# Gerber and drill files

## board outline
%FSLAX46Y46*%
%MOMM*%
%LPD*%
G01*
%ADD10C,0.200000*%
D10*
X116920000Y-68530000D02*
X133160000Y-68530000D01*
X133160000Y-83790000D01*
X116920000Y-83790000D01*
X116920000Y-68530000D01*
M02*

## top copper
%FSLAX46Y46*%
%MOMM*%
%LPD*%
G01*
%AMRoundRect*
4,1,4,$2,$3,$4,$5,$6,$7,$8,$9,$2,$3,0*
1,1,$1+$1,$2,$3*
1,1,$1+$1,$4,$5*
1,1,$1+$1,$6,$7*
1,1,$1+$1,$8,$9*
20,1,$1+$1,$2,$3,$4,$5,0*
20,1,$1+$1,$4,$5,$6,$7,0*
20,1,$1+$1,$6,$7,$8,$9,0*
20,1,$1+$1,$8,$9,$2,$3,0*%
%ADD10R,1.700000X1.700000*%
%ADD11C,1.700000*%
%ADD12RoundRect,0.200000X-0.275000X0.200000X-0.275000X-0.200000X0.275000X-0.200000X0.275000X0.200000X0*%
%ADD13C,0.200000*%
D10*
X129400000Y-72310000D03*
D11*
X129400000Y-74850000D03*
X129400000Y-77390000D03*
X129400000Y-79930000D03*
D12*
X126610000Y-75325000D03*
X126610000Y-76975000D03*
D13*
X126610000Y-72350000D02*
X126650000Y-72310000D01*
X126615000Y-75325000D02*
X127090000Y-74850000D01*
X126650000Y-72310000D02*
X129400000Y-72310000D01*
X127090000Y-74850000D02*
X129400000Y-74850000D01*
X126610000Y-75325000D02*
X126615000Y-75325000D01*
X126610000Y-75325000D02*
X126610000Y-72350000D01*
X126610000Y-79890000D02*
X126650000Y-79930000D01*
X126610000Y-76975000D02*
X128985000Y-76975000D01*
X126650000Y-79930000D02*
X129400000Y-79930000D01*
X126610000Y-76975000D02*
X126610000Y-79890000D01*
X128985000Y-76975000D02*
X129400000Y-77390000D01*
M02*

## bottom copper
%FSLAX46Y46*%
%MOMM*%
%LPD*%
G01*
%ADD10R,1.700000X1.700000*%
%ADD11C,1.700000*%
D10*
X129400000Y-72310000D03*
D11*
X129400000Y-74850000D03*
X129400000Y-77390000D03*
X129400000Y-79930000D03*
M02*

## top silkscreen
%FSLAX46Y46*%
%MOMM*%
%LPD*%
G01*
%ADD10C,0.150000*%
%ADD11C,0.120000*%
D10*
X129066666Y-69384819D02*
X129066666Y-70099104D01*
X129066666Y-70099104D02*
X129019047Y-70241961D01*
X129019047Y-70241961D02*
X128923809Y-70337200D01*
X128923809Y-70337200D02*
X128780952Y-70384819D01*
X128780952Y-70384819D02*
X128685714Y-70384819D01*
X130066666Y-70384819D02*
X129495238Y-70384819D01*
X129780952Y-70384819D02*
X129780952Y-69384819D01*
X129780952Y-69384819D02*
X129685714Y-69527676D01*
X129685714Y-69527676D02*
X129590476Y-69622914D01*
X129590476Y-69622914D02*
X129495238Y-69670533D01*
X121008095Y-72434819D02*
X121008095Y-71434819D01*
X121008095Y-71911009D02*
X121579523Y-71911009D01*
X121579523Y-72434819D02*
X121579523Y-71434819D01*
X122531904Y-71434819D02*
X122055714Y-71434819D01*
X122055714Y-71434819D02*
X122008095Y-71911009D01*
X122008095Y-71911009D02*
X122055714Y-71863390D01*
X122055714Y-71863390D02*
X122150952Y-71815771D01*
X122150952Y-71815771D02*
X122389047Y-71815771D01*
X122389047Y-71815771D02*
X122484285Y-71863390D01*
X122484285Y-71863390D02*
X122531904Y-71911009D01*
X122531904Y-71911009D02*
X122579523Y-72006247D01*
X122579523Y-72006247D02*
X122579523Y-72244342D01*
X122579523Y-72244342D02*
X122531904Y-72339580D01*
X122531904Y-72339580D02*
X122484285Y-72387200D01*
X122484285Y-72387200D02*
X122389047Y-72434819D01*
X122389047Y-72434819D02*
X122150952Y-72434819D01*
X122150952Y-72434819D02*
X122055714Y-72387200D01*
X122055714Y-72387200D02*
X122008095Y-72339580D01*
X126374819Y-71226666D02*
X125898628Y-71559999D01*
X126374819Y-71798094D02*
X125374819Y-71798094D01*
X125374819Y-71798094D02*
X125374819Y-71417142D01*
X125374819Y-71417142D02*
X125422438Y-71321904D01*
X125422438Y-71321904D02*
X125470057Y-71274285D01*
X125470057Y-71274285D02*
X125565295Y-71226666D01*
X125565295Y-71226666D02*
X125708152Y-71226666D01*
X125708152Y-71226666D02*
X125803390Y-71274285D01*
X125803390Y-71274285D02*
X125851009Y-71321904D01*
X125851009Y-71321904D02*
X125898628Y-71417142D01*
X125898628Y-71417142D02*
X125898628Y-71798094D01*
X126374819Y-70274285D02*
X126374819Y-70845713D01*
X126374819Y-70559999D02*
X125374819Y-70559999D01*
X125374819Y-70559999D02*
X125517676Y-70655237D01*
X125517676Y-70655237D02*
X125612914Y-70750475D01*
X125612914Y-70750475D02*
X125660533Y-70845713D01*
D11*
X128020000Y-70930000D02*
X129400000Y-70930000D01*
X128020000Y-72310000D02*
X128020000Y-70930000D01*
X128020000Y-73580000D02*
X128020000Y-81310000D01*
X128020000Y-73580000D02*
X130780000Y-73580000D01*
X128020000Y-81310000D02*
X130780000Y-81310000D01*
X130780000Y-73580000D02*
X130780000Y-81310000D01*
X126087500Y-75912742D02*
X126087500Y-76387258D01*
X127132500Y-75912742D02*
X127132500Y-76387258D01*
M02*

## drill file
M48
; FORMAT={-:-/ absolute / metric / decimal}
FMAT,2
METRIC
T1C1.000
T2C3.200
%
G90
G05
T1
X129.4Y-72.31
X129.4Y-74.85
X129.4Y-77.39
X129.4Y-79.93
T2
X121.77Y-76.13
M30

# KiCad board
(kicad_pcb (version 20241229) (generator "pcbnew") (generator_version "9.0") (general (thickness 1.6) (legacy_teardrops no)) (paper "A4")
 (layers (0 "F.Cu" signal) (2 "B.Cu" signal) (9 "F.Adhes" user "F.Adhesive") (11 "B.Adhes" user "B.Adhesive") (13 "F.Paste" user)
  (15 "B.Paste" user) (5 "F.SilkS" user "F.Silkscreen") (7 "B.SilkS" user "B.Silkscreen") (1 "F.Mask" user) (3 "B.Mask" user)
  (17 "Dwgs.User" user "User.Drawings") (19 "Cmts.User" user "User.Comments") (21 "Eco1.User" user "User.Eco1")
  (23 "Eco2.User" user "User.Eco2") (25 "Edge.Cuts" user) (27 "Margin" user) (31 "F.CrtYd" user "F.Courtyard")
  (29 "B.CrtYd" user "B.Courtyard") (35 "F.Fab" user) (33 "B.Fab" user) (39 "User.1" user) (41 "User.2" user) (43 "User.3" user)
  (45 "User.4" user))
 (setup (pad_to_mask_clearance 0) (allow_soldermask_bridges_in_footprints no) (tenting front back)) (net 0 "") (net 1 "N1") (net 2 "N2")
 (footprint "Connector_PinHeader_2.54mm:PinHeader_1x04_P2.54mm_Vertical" (layer "F.Cu") (at 129.4 72.31)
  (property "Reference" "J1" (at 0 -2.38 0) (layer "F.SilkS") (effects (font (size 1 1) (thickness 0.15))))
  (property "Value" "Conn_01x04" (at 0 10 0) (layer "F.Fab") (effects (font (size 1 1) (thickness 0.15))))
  (fp_line (start -1.38 -1.38) (end 0 -1.38) (stroke (width 0.12) (type solid)) (layer "F.SilkS"))
  (fp_line (start -1.38 0) (end -1.38 -1.38) (stroke (width 0.12) (type solid)) (layer "F.SilkS"))
  (fp_line (start -1.38 1.27) (end -1.38 9) (stroke (width 0.12) (type solid)) (layer "F.SilkS"))
  (fp_line (start -1.38 1.27) (end 1.38 1.27) (stroke (width 0.12) (type solid)) (layer "F.SilkS"))
  (fp_line (start -1.38 9) (end 1.38 9) (stroke (width 0.12) (type solid)) (layer "F.SilkS"))
  (fp_line (start 1.38 1.27) (end 1.38 9) (stroke (width 0.12) (type solid)) (layer "F.SilkS"))
  (pad "1" thru_hole rect (at 0 0) (size 1.7 1.7) (drill 1) (layers "*.Cu" "*.Mask") (remove_unused_layers no) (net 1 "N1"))
  (pad "2" thru_hole circle (at 0 2.54) (size 1.7 1.7) (drill 1) (layers "*.Cu" "*.Mask") (remove_unused_layers no) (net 1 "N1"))
  (pad "3" thru_hole circle (at 0 5.08) (size 1.7 1.7) (drill 1) (layers "*.Cu" "*.Mask") (remove_unused_layers no) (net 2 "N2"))
  (pad "4" thru_hole circle (at 0 7.62) (size 1.7 1.7) (drill 1) (layers "*.Cu" "*.Mask") (remove_unused_layers no) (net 2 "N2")))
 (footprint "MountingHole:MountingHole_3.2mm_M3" (layer "F.Cu") (at 121.77 76.13)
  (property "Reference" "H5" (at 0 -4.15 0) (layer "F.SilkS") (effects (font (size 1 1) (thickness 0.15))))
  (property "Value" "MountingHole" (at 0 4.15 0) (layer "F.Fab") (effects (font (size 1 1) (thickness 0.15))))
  (pad "" np_thru_hole circle (at 0 0) (size 3.2 3.2) (drill 3.2) (layers "*.Cu" "*.Mask")))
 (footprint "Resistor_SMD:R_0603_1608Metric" (layer "F.Cu") (at 126.61 76.15 -90)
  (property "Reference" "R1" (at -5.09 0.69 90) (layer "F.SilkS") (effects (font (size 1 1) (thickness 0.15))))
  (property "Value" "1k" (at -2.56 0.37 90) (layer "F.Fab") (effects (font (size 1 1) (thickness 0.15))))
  (fp_line (start -0.237258 0.5225) (end 0.237258 0.5225) (stroke (width 0.12) (type solid)) (layer "F.SilkS"))
  (fp_line (start -0.237258 -0.5225) (end 0.237258 -0.5225) (stroke (width 0.12) (type solid)) (layer "F.SilkS"))
  (pad "1" smd roundrect (at -0.825 0 270) (size 0.8 0.95) (layers "F.Cu" "F.Mask" "F.Paste") (roundrect_rratio 0.25) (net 1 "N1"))
  (pad "2" smd roundrect (at 0.825 0 270) (size 0.8 0.95) (layers "F.Cu" "F.Mask" "F.Paste") (roundrect_rratio 0.25) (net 2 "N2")))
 (gr_rect (start 116.92 68.53) (end 133.16 83.79) (stroke (width 0.2) (type solid)) (fill no) (layer "Edge.Cuts"))
 (segment (start 126.61 72.35) (end 126.65 72.31) (width 0.2) (layer "F.Cu") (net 1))
 (segment (start 126.615 75.325) (end 127.09 74.85) (width 0.2) (layer "F.Cu") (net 1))
 (segment (start 126.65 72.31) (end 129.4 72.31) (width 0.2) (layer "F.Cu") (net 1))
 (segment (start 127.09 74.85) (end 129.4 74.85) (width 0.2) (layer "F.Cu") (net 1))
 (segment (start 126.61 75.325) (end 126.615 75.325) (width 0.2) (layer "F.Cu") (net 1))
 (segment (start 126.61 75.325) (end 126.61 72.35) (width 0.2) (layer "F.Cu") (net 1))
 (segment (start 126.61 79.89) (end 126.65 79.93) (width 0.2) (layer "F.Cu") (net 2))
 (segment (start 126.61 76.975) (end 128.985 76.975) (width 0.2) (layer "F.Cu") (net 2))
 (segment (start 126.65 79.93) (end 129.4 79.93) (width 0.2) (layer "F.Cu") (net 2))
 (segment (start 126.61 76.975) (end 126.61 79.89) (width 0.2) (layer "F.Cu") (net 2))
 (segment (start 128.985 76.975) (end 129.4 77.39) (width 0.2) (layer "F.Cu") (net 2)))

